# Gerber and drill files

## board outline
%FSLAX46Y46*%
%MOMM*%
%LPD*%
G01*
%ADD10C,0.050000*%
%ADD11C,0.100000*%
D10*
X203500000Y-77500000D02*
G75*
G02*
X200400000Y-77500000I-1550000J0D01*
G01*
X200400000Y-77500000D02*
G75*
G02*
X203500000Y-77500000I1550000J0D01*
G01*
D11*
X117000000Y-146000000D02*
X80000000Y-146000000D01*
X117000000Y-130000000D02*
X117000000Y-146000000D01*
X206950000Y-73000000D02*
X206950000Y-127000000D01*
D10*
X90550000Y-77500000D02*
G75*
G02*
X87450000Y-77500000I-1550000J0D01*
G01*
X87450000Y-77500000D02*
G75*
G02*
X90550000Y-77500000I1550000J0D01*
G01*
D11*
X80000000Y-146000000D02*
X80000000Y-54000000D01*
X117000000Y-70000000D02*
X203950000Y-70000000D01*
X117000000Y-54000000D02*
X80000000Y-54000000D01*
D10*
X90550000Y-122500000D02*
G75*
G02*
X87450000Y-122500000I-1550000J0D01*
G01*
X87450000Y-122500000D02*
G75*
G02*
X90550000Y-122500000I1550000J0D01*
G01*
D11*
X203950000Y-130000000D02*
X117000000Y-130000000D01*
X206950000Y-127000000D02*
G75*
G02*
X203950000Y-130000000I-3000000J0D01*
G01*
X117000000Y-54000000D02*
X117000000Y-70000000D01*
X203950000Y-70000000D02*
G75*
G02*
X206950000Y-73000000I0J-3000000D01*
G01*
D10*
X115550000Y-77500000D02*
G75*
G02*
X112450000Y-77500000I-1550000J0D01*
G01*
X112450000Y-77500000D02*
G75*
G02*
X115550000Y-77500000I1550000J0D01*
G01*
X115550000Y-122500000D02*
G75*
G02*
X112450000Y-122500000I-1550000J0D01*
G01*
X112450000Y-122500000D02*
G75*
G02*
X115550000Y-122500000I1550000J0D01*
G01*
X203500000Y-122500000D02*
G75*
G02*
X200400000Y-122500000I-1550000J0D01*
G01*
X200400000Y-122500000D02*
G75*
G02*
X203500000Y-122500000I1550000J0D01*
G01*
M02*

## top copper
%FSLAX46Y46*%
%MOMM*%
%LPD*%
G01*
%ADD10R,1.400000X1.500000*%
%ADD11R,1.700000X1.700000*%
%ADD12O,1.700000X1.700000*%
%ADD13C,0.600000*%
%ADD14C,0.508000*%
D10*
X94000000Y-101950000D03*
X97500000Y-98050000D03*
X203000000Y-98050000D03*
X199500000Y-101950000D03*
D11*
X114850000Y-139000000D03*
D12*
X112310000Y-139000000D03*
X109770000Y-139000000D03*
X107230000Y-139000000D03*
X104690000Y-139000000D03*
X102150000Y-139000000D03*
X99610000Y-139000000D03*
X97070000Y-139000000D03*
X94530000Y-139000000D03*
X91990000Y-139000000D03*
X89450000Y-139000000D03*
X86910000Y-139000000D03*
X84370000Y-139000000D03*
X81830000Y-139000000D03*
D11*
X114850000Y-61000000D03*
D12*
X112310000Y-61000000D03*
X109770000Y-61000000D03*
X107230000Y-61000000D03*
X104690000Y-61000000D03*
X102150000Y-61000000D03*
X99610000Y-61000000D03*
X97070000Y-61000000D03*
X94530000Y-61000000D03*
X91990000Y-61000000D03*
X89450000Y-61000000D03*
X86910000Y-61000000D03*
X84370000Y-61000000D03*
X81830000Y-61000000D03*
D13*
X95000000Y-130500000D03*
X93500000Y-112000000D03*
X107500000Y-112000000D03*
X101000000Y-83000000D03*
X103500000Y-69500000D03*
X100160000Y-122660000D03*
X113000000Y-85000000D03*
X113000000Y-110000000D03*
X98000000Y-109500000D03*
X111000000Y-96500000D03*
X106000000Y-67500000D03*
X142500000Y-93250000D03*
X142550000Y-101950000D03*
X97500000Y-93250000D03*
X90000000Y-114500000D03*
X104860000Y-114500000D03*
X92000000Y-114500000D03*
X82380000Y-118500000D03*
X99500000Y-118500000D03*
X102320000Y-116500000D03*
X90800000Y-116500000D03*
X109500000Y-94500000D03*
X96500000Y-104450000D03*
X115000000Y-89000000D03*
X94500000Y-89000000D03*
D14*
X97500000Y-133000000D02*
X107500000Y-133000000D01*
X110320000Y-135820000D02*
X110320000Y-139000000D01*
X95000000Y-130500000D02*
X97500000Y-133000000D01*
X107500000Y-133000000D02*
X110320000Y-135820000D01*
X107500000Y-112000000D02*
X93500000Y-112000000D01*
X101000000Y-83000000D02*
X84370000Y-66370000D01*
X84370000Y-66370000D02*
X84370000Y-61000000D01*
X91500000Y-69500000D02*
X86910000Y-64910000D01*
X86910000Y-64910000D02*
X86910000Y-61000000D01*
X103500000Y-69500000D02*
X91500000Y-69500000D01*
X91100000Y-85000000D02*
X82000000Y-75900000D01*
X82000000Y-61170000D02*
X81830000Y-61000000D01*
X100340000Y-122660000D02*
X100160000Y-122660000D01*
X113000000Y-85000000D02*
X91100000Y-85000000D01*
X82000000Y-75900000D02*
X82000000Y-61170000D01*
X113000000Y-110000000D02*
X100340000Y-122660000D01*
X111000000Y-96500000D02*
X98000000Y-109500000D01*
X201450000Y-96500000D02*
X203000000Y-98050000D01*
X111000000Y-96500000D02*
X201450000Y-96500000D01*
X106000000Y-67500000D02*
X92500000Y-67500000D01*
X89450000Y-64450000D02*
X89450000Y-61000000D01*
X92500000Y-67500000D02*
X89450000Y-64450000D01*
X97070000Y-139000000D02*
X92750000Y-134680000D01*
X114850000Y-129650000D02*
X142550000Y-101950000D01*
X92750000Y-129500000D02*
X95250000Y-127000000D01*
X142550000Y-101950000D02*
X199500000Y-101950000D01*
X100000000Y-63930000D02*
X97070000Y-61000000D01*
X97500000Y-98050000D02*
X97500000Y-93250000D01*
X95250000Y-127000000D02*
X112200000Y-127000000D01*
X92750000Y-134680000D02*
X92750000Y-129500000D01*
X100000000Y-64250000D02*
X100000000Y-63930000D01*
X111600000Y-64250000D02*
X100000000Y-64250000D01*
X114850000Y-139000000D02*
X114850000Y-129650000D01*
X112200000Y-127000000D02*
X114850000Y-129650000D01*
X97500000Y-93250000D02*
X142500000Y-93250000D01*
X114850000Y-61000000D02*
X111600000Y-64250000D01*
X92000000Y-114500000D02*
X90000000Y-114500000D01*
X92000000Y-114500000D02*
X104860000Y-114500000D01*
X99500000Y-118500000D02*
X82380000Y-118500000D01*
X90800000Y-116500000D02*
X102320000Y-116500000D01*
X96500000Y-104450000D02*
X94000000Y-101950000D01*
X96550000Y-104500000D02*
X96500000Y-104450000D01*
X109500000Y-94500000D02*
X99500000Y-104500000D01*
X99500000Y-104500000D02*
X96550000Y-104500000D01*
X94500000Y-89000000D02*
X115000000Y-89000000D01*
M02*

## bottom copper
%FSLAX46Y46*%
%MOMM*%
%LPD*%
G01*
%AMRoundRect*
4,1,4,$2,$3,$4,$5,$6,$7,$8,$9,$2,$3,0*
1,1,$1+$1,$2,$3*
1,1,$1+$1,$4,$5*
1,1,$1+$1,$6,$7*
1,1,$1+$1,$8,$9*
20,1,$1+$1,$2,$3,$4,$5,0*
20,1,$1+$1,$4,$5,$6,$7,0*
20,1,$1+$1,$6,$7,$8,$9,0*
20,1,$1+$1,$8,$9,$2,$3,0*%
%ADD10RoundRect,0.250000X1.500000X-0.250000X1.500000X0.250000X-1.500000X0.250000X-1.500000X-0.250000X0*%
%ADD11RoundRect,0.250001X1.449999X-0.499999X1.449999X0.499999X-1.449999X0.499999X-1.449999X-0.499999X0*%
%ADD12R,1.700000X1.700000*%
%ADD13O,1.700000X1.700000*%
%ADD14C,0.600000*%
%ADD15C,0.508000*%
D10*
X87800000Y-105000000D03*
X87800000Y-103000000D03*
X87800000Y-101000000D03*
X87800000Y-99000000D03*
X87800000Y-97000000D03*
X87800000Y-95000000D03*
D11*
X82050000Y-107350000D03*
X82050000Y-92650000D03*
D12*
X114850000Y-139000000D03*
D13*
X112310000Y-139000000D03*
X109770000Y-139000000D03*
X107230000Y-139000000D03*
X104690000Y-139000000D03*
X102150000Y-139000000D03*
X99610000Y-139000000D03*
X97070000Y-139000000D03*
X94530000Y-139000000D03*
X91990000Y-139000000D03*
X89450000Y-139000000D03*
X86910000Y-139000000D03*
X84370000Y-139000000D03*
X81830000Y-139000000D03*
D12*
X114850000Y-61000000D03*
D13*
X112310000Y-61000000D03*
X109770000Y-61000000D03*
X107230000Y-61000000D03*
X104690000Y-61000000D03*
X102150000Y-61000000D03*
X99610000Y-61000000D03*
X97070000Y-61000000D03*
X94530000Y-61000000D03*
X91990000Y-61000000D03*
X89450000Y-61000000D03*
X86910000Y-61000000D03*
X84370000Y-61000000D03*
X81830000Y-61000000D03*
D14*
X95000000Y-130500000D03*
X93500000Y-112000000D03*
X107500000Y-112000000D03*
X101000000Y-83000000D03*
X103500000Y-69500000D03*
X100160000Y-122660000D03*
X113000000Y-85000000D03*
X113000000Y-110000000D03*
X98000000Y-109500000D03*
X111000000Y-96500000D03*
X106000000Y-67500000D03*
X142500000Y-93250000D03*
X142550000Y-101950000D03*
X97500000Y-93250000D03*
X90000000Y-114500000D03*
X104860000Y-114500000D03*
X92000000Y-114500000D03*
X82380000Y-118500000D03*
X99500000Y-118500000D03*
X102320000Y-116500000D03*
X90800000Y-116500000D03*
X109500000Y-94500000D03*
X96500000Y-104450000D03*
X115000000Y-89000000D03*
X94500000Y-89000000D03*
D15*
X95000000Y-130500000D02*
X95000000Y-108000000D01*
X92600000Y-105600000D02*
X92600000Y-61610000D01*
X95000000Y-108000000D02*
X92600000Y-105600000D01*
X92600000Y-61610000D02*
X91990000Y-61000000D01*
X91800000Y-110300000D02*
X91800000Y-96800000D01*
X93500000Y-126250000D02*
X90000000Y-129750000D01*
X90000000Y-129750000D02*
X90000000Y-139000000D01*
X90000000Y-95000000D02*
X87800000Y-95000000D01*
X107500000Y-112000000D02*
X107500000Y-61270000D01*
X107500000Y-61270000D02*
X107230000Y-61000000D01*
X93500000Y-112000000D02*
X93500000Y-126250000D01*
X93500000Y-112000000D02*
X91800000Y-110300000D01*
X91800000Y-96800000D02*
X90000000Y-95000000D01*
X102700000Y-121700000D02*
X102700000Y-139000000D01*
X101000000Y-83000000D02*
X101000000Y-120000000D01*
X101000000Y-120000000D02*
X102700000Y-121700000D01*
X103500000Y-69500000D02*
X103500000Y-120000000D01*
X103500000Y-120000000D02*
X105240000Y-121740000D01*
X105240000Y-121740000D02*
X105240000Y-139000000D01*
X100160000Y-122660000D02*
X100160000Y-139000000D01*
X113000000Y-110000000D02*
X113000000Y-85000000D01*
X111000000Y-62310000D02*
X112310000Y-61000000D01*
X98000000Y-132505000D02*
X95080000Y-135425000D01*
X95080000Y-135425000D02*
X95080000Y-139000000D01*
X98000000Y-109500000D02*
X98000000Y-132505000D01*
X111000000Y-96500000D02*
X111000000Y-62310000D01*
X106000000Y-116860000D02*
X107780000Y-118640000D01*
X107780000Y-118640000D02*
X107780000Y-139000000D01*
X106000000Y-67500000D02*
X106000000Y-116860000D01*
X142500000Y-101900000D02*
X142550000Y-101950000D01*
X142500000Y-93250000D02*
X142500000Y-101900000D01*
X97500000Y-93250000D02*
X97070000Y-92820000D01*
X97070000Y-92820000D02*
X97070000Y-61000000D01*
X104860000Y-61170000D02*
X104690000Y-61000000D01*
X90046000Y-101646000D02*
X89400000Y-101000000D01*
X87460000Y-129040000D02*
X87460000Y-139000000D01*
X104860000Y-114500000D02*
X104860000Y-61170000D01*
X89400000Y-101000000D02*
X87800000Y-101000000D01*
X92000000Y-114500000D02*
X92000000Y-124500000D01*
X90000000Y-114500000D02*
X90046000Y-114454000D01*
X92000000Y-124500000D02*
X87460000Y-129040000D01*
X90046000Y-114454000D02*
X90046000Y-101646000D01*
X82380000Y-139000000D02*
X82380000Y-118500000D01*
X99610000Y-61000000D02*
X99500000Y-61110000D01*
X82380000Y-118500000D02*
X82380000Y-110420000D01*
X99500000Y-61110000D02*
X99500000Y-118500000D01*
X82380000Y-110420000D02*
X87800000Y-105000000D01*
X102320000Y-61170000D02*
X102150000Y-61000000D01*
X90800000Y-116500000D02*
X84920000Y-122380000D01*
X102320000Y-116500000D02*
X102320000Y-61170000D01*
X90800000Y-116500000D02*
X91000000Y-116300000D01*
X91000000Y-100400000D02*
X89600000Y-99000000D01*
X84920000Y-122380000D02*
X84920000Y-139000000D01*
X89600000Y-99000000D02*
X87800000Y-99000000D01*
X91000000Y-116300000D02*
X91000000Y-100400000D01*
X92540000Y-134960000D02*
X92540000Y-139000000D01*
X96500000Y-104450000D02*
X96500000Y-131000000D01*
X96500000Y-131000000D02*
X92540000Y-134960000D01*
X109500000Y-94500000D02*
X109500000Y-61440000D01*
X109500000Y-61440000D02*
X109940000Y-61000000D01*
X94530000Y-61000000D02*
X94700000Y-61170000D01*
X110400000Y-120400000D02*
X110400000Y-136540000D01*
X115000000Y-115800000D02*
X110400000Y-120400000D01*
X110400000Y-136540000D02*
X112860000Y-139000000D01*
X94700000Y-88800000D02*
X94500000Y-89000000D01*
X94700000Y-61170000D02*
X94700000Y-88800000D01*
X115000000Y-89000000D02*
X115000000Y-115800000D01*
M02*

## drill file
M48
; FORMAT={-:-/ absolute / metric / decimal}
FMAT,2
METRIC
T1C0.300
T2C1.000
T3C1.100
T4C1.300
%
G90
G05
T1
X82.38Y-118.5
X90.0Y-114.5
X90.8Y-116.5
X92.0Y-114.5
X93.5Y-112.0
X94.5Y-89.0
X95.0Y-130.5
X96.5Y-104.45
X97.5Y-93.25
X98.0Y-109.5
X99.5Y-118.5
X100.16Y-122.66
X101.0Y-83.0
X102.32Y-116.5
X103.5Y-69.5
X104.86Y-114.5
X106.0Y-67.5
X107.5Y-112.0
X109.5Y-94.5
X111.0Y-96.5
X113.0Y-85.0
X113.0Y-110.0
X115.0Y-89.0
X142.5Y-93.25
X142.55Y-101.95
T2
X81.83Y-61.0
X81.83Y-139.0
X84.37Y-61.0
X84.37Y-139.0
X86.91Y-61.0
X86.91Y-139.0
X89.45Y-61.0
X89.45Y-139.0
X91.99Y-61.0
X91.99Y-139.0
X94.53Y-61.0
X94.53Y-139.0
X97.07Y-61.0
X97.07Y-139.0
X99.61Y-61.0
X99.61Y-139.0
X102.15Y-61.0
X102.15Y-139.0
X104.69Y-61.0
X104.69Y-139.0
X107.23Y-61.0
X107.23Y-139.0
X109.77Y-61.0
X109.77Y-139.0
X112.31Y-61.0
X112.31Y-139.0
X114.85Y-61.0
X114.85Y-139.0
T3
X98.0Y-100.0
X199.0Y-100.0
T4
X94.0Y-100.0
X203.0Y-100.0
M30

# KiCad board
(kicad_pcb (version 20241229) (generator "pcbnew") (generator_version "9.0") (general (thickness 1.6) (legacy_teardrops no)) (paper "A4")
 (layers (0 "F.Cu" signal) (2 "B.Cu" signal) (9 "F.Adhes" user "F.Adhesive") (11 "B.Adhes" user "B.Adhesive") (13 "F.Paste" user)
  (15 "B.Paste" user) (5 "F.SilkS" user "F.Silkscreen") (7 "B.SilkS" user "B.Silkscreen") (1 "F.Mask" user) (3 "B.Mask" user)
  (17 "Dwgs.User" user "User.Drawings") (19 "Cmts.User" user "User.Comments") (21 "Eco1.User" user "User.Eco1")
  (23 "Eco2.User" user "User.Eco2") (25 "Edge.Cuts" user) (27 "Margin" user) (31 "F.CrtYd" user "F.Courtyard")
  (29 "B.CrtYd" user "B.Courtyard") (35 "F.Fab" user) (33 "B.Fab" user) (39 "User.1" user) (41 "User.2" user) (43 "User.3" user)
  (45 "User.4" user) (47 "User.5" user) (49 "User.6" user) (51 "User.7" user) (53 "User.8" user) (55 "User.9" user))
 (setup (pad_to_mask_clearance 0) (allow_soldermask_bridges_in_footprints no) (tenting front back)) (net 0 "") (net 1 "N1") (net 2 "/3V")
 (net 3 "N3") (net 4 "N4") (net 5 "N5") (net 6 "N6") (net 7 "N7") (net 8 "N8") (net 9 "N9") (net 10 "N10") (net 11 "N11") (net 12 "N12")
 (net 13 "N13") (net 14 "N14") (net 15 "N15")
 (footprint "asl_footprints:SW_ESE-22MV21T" (layer "F.Cu") (at 96 100 180)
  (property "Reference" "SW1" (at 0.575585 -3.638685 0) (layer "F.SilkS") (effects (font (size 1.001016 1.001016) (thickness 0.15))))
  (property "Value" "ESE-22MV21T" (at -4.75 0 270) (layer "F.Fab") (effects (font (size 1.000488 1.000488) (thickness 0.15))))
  (pad "" np_thru_hole circle (at -2 0 180) (size 1.1 1.1) (drill 1.1) (layers "*.Cu" "*.Mask"))
  (pad "" np_thru_hole circle (at 2 0 180) (size 1.3 1.3) (drill 1.3) (layers "*.Cu" "*.Mask"))
  (pad "1" smd rect (at 2 -1.95 180) (size 1.4 1.5) (layers "F.Cu" "F.Mask" "F.Paste") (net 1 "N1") (solder_mask_margin 0.102))
  (pad "2" smd rect (at -1.5 1.95 180) (size 1.4 1.5) (layers "F.Cu" "F.Mask" "F.Paste") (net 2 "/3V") (solder_mask_margin 0.102)))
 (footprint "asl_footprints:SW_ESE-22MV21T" (layer "F.Cu") (at 201 100)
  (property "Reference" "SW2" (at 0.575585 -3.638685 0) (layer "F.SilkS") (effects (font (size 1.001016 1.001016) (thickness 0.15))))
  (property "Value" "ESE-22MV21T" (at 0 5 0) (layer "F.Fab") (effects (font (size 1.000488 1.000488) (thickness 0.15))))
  (pad "" np_thru_hole circle (at -2 0) (size 1.1 1.1) (drill 1.1) (layers "*.Cu" "*.Mask"))
  (pad "" np_thru_hole circle (at 2 0) (size 1.3 1.3) (drill 1.3) (layers "*.Cu" "*.Mask"))
  (pad "1" smd rect (at 2 -1.95) (size 1.4 1.5) (layers "F.Cu" "F.Mask" "F.Paste") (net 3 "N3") (solder_mask_margin 0.102))
  (pad "2" smd rect (at -1.5 1.95) (size 1.4 1.5) (layers "F.Cu" "F.Mask" "F.Paste") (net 2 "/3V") (solder_mask_margin 0.102)))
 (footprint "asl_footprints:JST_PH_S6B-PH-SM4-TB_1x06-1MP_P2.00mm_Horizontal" (layer "B.Cu") (at 84.95 100 90)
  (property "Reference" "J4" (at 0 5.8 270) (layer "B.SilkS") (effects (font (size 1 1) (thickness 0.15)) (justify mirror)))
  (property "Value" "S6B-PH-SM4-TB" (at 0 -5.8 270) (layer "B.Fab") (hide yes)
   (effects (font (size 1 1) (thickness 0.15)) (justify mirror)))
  (pad "1" smd roundrect (at -5 2.85 90) (size 1 3.5) (layers "B.Cu" "B.Mask" "B.Paste") (roundrect_rratio 0.25) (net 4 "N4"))
  (pad "2" smd roundrect (at -3 2.85 90) (size 1 3.5) (layers "B.Cu" "B.Mask" "B.Paste") (roundrect_rratio 0.25) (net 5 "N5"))
  (pad "3" smd roundrect (at -1 2.85 90) (size 1 3.5) (layers "B.Cu" "B.Mask" "B.Paste") (roundrect_rratio 0.25) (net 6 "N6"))
  (pad "4" smd roundrect (at 1 2.85 90) (size 1 3.5) (layers "B.Cu" "B.Mask" "B.Paste") (roundrect_rratio 0.25) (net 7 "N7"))
  (pad "5" smd roundrect (at 3 2.85 90) (size 1 3.5) (layers "B.Cu" "B.Mask" "B.Paste") (roundrect_rratio 0.25) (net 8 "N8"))
  (pad "6" smd roundrect (at 5 2.85 90) (size 1 3.5) (layers "B.Cu" "B.Mask" "B.Paste") (roundrect_rratio 0.25) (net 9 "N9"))
  (pad "MP" smd roundrect (at -7.35 -2.9 90) (size 1.5 3.4) (layers "B.Cu" "B.Mask" "B.Paste") (roundrect_rratio 0.166667))
  (pad "MP" smd roundrect (at 7.35 -2.9 90) (size 1.5 3.4) (layers "B.Cu" "B.Mask" "B.Paste") (roundrect_rratio 0.166667)))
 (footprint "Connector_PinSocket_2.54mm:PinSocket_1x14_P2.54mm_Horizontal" (layer "B.Cu") (at 114.85 139 90)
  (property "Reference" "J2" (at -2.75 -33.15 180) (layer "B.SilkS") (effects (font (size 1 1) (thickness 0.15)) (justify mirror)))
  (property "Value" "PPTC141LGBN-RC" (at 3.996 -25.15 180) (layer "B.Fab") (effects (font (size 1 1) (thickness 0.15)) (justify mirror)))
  (pad "1" thru_hole rect (at 0 0 90) (size 1.7 1.7) (drill 1) (layers "*.Cu" "*.Mask") (remove_unused_layers no) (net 2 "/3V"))
  (pad "2" thru_hole oval (at 0 -2.54 90) (size 1.7 1.7) (drill 1) (layers "*.Cu" "*.Mask") (remove_unused_layers no) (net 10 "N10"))
  (pad "3" thru_hole oval (at 0 -5.08 90) (size 1.7 1.7) (drill 1) (layers "*.Cu" "*.Mask") (remove_unused_layers no) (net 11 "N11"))
  (pad "4" thru_hole oval (at 0 -7.62 90) (size 1.7 1.7) (drill 1) (layers "*.Cu" "*.Mask") (remove_unused_layers no) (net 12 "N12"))
  (pad "5" thru_hole oval (at 0 -10.16 90) (size 1.7 1.7) (drill 1) (layers "*.Cu" "*.Mask") (remove_unused_layers no) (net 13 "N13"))
  (pad "6" thru_hole oval (at 0 -12.7 90) (size 1.7 1.7) (drill 1) (layers "*.Cu" "*.Mask") (remove_unused_layers no) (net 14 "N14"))
  (pad "7" thru_hole oval (at 0 -15.24 90) (size 1.7 1.7) (drill 1) (layers "*.Cu" "*.Mask") (remove_unused_layers no) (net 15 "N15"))
  (pad "8" thru_hole oval (at 0 -17.78 90) (size 1.7 1.7) (drill 1) (layers "*.Cu" "*.Mask") (remove_unused_layers no) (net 2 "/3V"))
  (pad "9" thru_hole oval (at 0 -20.32 90) (size 1.7 1.7) (drill 1) (layers "*.Cu" "*.Mask") (remove_unused_layers no) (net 3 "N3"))
  (pad "10" thru_hole oval (at 0 -22.86 90) (size 1.7 1.7) (drill 1) (layers "*.Cu" "*.Mask") (remove_unused_layers no) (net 1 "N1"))
  (pad "11" thru_hole oval (at 0 -25.4 90) (size 1.7 1.7) (drill 1) (layers "*.Cu" "*.Mask") (remove_unused_layers no) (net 9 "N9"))
  (pad "12" thru_hole oval (at 0 -27.94 90) (size 1.7 1.7) (drill 1) (layers "*.Cu" "*.Mask") (remove_unused_layers no) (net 6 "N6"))
  (pad "13" thru_hole oval (at 0 -30.48 90) (size 1.7 1.7) (drill 1) (layers "*.Cu" "*.Mask") (remove_unused_layers no) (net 7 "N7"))
  (pad "14" thru_hole oval (at 0 -33.02 90) (size 1.7 1.7) (drill 1) (layers "*.Cu" "*.Mask") (remove_unused_layers no) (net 4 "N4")))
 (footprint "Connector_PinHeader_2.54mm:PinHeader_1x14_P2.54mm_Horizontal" (layer "B.Cu") (at 114.85 61 90)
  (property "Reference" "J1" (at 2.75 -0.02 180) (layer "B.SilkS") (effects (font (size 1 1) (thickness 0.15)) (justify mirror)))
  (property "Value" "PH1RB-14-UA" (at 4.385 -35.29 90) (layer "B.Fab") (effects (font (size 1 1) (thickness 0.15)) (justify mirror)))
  (pad "1" thru_hole rect (at 0 0 90) (size 1.7 1.7) (drill 1) (layers "*.Cu" "*.Mask") (remove_unused_layers no) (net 2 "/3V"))
  (pad "2" thru_hole oval (at 0 -2.54 90) (size 1.7 1.7) (drill 1) (layers "*.Cu" "*.Mask") (remove_unused_layers no) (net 3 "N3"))
  (pad "3" thru_hole oval (at 0 -5.08 90) (size 1.7 1.7) (drill 1) (layers "*.Cu" "*.Mask") (remove_unused_layers no) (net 1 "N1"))
  (pad "4" thru_hole oval (at 0 -7.62 90) (size 1.7 1.7) (drill 1) (layers "*.Cu" "*.Mask") (remove_unused_layers no) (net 9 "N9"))
  (pad "5" thru_hole oval (at 0 -10.16 90) (size 1.7 1.7) (drill 1) (layers "*.Cu" "*.Mask") (remove_unused_layers no) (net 6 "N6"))
  (pad "6" thru_hole oval (at 0 -12.7 90) (size 1.7 1.7) (drill 1) (layers "*.Cu" "*.Mask") (remove_unused_layers no) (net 7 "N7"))
  (pad "7" thru_hole oval (at 0 -15.24 90) (size 1.7 1.7) (drill 1) (layers "*.Cu" "*.Mask") (remove_unused_layers no) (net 4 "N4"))
  (pad "8" thru_hole oval (at 0 -17.78 90) (size 1.7 1.7) (drill 1) (layers "*.Cu" "*.Mask") (remove_unused_layers no) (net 2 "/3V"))
  (pad "9" thru_hole oval (at 0 -20.32 90) (size 1.7 1.7) (drill 1) (layers "*.Cu" "*.Mask") (remove_unused_layers no) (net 10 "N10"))
  (pad "10" thru_hole oval (at 0 -22.86 90) (size 1.7 1.7) (drill 1) (layers "*.Cu" "*.Mask") (remove_unused_layers no) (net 11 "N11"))
  (pad "11" thru_hole oval (at 0 -25.4 90) (size 1.7 1.7) (drill 1) (layers "*.Cu" "*.Mask") (remove_unused_layers no) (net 12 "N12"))
  (pad "12" thru_hole oval (at 0 -27.94 90) (size 1.7 1.7) (drill 1) (layers "*.Cu" "*.Mask") (remove_unused_layers no) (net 13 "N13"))
  (pad "13" thru_hole oval (at 0 -30.48 90) (size 1.7 1.7) (drill 1) (layers "*.Cu" "*.Mask") (remove_unused_layers no) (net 14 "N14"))
  (pad "14" thru_hole oval (at 0 -33.02 90) (size 1.7 1.7) (drill 1) (layers "*.Cu" "*.Mask") (remove_unused_layers no) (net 15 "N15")))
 (gr_circle (center 201.95 77.5) (end 203.5 77.5) (stroke (width 0.05) (type default)) (fill no) (layer "Edge.Cuts"))
 (gr_line (start 117 146) (end 80 146) (stroke (width 0.1) (type default)) (layer "Edge.Cuts"))
 (gr_line (start 117 130) (end 117 146) (stroke (width 0.1) (type default)) (layer "Edge.Cuts"))
 (gr_line (start 206.95 73) (end 206.95 127) (stroke (width 0.1) (type default)) (layer "Edge.Cuts"))
 (gr_circle (center 89 77.5) (end 90.55 77.5) (stroke (width 0.05) (type default)) (fill no) (layer "Edge.Cuts"))
 (gr_line (start 80 146) (end 80 54) (stroke (width 0.1) (type default)) (layer "Edge.Cuts"))
 (gr_line (start 117 70) (end 203.95 70) (stroke (width 0.1) (type default)) (layer "Edge.Cuts"))
 (gr_line (start 117 54) (end 80 54) (stroke (width 0.1) (type default)) (layer "Edge.Cuts"))
 (gr_circle (center 89 122.5) (end 90.55 122.5) (stroke (width 0.05) (type default)) (fill no) (layer "Edge.Cuts"))
 (gr_line (start 203.95 130) (end 117 130) (stroke (width 0.1) (type default)) (layer "Edge.Cuts"))
 (gr_arc (start 206.95 127) (mid 206.07132 129.12132) (end 203.95 130) (stroke (width 0.1) (type default)) (layer "Edge.Cuts"))
 (gr_line (start 117 54) (end 117 70) (stroke (width 0.1) (type default)) (layer "Edge.Cuts"))
 (gr_arc (start 203.95 70) (mid 206.07132 70.87868) (end 206.95 73) (stroke (width 0.1) (type default)) (layer "Edge.Cuts"))
 (gr_circle (center 114 77.5) (end 115.55 77.5) (stroke (width 0.05) (type default)) (fill no) (layer "Edge.Cuts"))
 (gr_circle (center 114 122.5) (end 115.55 122.5) (stroke (width 0.05) (type default)) (fill no) (layer "Edge.Cuts"))
 (gr_circle (center 201.95 122.5) (end 203.5 122.5) (stroke (width 0.05) (type default)) (fill no) (layer "Edge.Cuts"))
 (segment (start 97.5 133) (end 107.5 133) (width 0.508) (layer "F.Cu") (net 11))
 (segment (start 110.32 135.82) (end 110.32 139) (width 0.508) (layer "F.Cu") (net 11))
 (segment (start 95 130.5) (end 97.5 133) (width 0.508) (layer "F.Cu") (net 11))
 (segment (start 107.5 133) (end 110.32 135.82) (width 0.508) (layer "F.Cu") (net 11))
 (via (at 95 130.5) (size 0.6) (drill 0.3) (layers "F.Cu" "B.Cu") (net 11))
 (segment (start 95 130.5) (end 95 108) (width 0.508) (layer "B.Cu") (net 11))
 (segment (start 92.6 105.6) (end 92.6 61.61) (width 0.508) (layer "B.Cu") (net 11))
 (segment (start 95 108) (end 92.6 105.6) (width 0.508) (layer "B.Cu") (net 11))
 (segment (start 92.6 61.61) (end 91.99 61) (width 0.508) (layer "B.Cu") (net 11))
 (segment (start 107.5 112) (end 93.5 112) (width 0.508) (layer "F.Cu") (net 9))
 (via (at 93.5 112) (size 0.6) (drill 0.3) (layers "F.Cu" "B.Cu") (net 9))
 (via (at 107.5 112) (size 0.6) (drill 0.3) (layers "F.Cu" "B.Cu") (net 9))
 (segment (start 91.8 110.3) (end 91.8 96.8) (width 0.508) (layer "B.Cu") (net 9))
 (segment (start 93.5 126.25) (end 90 129.75) (width 0.508) (layer "B.Cu") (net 9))
 (segment (start 90 129.75) (end 90 139) (width 0.508) (layer "B.Cu") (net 9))
 (segment (start 90 95) (end 87.8 95) (width 0.508) (layer "B.Cu") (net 9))
 (segment (start 107.5 112) (end 107.5 61.27) (width 0.508) (layer "B.Cu") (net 9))
 (segment (start 107.5 61.27) (end 107.23 61) (width 0.508) (layer "B.Cu") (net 9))
 (segment (start 93.5 112) (end 93.5 126.25) (width 0.508) (layer "B.Cu") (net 9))
 (segment (start 93.5 112) (end 91.8 110.3) (width 0.508) (layer "B.Cu") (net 9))
 (segment (start 91.8 96.8) (end 90 95) (width 0.508) (layer "B.Cu") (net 9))
 (segment (start 101 83) (end 84.37 66.37) (width 0.508) (layer "F.Cu") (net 14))
 (segment (start 84.37 66.37) (end 84.37 61) (width 0.508) (layer "F.Cu") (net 14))
 (via (at 101 83) (size 0.6) (drill 0.3) (layers "F.Cu" "B.Cu") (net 14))
 (segment (start 102.7 121.7) (end 102.7 139) (width 0.508) (layer "B.Cu") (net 14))
 (segment (start 101 83) (end 101 120) (width 0.508) (layer "B.Cu") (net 14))
 (segment (start 101 120) (end 102.7 121.7) (width 0.508) (layer "B.Cu") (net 14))
 (segment (start 91.5 69.5) (end 86.91 64.91) (width 0.508) (layer "F.Cu") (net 13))
 (segment (start 86.91 64.91) (end 86.91 61) (width 0.508) (layer "F.Cu") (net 13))
 (segment (start 103.5 69.5) (end 91.5 69.5) (width 0.508) (layer "F.Cu") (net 13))
 (via (at 103.5 69.5) (size 0.6) (drill 0.3) (layers "F.Cu" "B.Cu") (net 13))
 (segment (start 103.5 69.5) (end 103.5 120) (width 0.508) (layer "B.Cu") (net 13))
 (segment (start 103.5 120) (end 105.24 121.74) (width 0.508) (layer "B.Cu") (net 13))
 (segment (start 105.24 121.74) (end 105.24 139) (width 0.508) (layer "B.Cu") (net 13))
 (segment (start 91.1 85) (end 82 75.9) (width 0.508) (layer "F.Cu") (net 15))
 (segment (start 82 61.17) (end 81.83 61) (width 0.508) (layer "F.Cu") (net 15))
 (segment (start 100.34 122.66) (end 100.16 122.66) (width 0.508) (layer "F.Cu") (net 15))
 (segment (start 113 85) (end 91.1 85) (width 0.508) (layer "F.Cu") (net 15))
 (segment (start 82 75.9) (end 82 61.17) (width 0.508) (layer "F.Cu") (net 15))
 (segment (start 113 110) (end 100.34 122.66) (width 0.508) (layer "F.Cu") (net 15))
 (via (at 100.16 122.66) (size 0.6) (drill 0.3) (layers "F.Cu" "B.Cu") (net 15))
 (via (at 113 85) (size 0.6) (drill 0.3) (layers "F.Cu" "B.Cu") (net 15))
 (via (at 113 110) (size 0.6) (drill 0.3) (layers "F.Cu" "B.Cu") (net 15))
 (segment (start 100.16 122.66) (end 100.16 139) (width 0.508) (layer "B.Cu") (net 15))
 (segment (start 113 110) (end 113 85) (width 0.508) (layer "B.Cu") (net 15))
 (segment (start 111 96.5) (end 98 109.5) (width 0.508) (layer "F.Cu") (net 3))
 (segment (start 201.45 96.5) (end 203 98.05) (width 0.508) (layer "F.Cu") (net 3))
 (segment (start 111 96.5) (end 201.45 96.5) (width 0.508) (layer "F.Cu") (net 3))
 (via (at 98 109.5) (size 0.6) (drill 0.3) (layers "F.Cu" "B.Cu") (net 3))
 (via (at 111 96.5) (size 0.6) (drill 0.3) (layers "F.Cu" "B.Cu") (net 3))
 (segment (start 111 62.31) (end 112.31 61) (width 0.508) (layer "B.Cu") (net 3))
 (segment (start 98 132.505) (end 95.08 135.425) (width 0.508) (layer "B.Cu") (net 3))
 (segment (start 95.08 135.425) (end 95.08 139) (width 0.508) (layer "B.Cu") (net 3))
 (segment (start 98 109.5) (end 98 132.505) (width 0.508) (layer "B.Cu") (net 3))
 (segment (start 111 96.5) (end 111 62.31) (width 0.508) (layer "B.Cu") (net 3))
 (segment (start 106 67.5) (end 92.5 67.5) (width 0.508) (layer "F.Cu") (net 12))
 (segment (start 89.45 64.45) (end 89.45 61) (width 0.508) (layer "F.Cu") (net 12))
 (segment (start 92.5 67.5) (end 89.45 64.45) (width 0.508) (layer "F.Cu") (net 12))
 (via (at 106 67.5) (size 0.6) (drill 0.3) (layers "F.Cu" "B.Cu") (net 12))
 (segment (start 106 116.86) (end 107.78 118.64) (width 0.508) (layer "B.Cu") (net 12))
 (segment (start 107.78 118.64) (end 107.78 139) (width 0.508) (layer "B.Cu") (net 12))
 (segment (start 106 67.5) (end 106 116.86) (width 0.508) (layer "B.Cu") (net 12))
 (segment (start 97.07 139) (end 92.75 134.68) (width 0.508) (layer "F.Cu") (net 2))
 (segment (start 114.85 129.65) (end 142.55 101.95) (width 0.508) (layer "F.Cu") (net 2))
 (segment (start 92.75 129.5) (end 95.25 127) (width 0.508) (layer "F.Cu") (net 2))
 (segment (start 142.55 101.95) (end 199.5 101.95) (width 0.508) (layer "F.Cu") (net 2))
 (segment (start 100 63.93) (end 97.07 61) (width 0.508) (layer "F.Cu") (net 2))
 (segment (start 97.5 98.05) (end 97.5 93.25) (width 0.508) (layer "F.Cu") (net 2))
 (segment (start 95.25 127) (end 112.2 127) (width 0.508) (layer "F.Cu") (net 2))
 (segment (start 92.75 134.68) (end 92.75 129.5) (width 0.508) (layer "F.Cu") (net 2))
 (segment (start 100 64.25) (end 100 63.93) (width 0.508) (layer "F.Cu") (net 2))
 (segment (start 111.6 64.25) (end 100 64.25) (width 0.508) (layer "F.Cu") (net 2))
 (segment (start 114.85 139) (end 114.85 129.65) (width 0.508) (layer "F.Cu") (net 2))
 (segment (start 112.2 127) (end 114.85 129.65) (width 0.508) (layer "F.Cu") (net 2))
 (segment (start 97.5 93.25) (end 142.5 93.25) (width 0.508) (layer "F.Cu") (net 2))
 (segment (start 114.85 61) (end 111.6 64.25) (width 0.508) (layer "F.Cu") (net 2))
 (via (at 142.5 93.25) (size 0.6) (drill 0.3) (layers "F.Cu" "B.Cu") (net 2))
 (via (at 142.55 101.95) (size 0.6) (drill 0.3) (layers "F.Cu" "B.Cu") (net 2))
 (via (at 97.5 93.25) (size 0.6) (drill 0.3) (layers "F.Cu" "B.Cu") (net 2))
 (segment (start 142.5 101.9) (end 142.55 101.95) (width 0.508) (layer "B.Cu") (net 2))
 (segment (start 142.5 93.25) (end 142.5 101.9) (width 0.508) (layer "B.Cu") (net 2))
 (segment (start 97.5 93.25) (end 97.07 92.82) (width 0.508) (layer "B.Cu") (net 2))
 (segment (start 97.07 92.82) (end 97.07 61) (width 0.508) (layer "B.Cu") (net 2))
 (segment (start 92 114.5) (end 90 114.5) (width 0.508) (layer "F.Cu") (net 6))
 (segment (start 92 114.5) (end 104.86 114.5) (width 0.508) (layer "F.Cu") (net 6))
 (via (at 90 114.5) (size 0.6) (drill 0.3) (layers "F.Cu" "B.Cu") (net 6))
 (via (at 104.86 114.5) (size 0.6) (drill 0.3) (layers "F.Cu" "B.Cu") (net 6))
 (via (at 92 114.5) (size 0.6) (drill 0.3) (layers "F.Cu" "B.Cu") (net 6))
 (segment (start 104.86 61.17) (end 104.69 61) (width 0.508) (layer "B.Cu") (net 6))
 (segment (start 90.046 101.646) (end 89.4 101) (width 0.508) (layer "B.Cu") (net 6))
 (segment (start 87.46 129.04) (end 87.46 139) (width 0.508) (layer "B.Cu") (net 6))
 (segment (start 104.86 114.5) (end 104.86 61.17) (width 0.508) (layer "B.Cu") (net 6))
 (segment (start 89.4 101) (end 87.8 101) (width 0.508) (layer "B.Cu") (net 6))
 (segment (start 92 114.5) (end 92 124.5) (width 0.508) (layer "B.Cu") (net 6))
 (segment (start 90 114.5) (end 90.046 114.454) (width 0.508) (layer "B.Cu") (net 6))
 (segment (start 92 124.5) (end 87.46 129.04) (width 0.508) (layer "B.Cu") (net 6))
 (segment (start 90.046 114.454) (end 90.046 101.646) (width 0.508) (layer "B.Cu") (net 6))
 (segment (start 99.5 118.5) (end 82.38 118.5) (width 0.508) (layer "F.Cu") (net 4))
 (via (at 82.38 118.5) (size 0.6) (drill 0.3) (layers "F.Cu" "B.Cu") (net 4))
 (via (at 99.5 118.5) (size 0.6) (drill 0.3) (layers "F.Cu" "B.Cu") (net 4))
 (segment (start 82.38 139) (end 82.38 118.5) (width 0.508) (layer "B.Cu") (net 4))
 (segment (start 99.61 61) (end 99.5 61.11) (width 0.508) (layer "B.Cu") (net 4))
 (segment (start 82.38 118.5) (end 82.38 110.42) (width 0.508) (layer "B.Cu") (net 4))
 (segment (start 99.5 61.11) (end 99.5 118.5) (width 0.508) (layer "B.Cu") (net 4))
 (segment (start 82.38 110.42) (end 87.8 105) (width 0.508) (layer "B.Cu") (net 4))
 (segment (start 90.8 116.5) (end 102.32 116.5) (width 0.508) (layer "F.Cu") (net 7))
 (via (at 102.32 116.5) (size 0.6) (drill 0.3) (layers "F.Cu" "B.Cu") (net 7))
 (via (at 90.8 116.5) (size 0.6) (drill 0.3) (layers "F.Cu" "B.Cu") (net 7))
 (segment (start 102.32 61.17) (end 102.15 61) (width 0.508) (layer "B.Cu") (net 7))
 (segment (start 90.8 116.5) (end 84.92 122.38) (width 0.508) (layer "B.Cu") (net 7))
 (segment (start 102.32 116.5) (end 102.32 61.17) (width 0.508) (layer "B.Cu") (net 7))
 (segment (start 90.8 116.5) (end 91 116.3) (width 0.508) (layer "B.Cu") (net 7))
 (segment (start 91 100.4) (end 89.6 99) (width 0.508) (layer "B.Cu") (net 7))
 (segment (start 84.92 122.38) (end 84.92 139) (width 0.508) (layer "B.Cu") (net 7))
 (segment (start 89.6 99) (end 87.8 99) (width 0.508) (layer "B.Cu") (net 7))
 (segment (start 91 116.3) (end 91 100.4) (width 0.508) (layer "B.Cu") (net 7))
 (segment (start 96.5 104.45) (end 94 101.95) (width 0.508) (layer "F.Cu") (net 1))
 (segment (start 96.55 104.5) (end 96.5 104.45) (width 0.508) (layer "F.Cu") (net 1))
 (segment (start 109.5 94.5) (end 99.5 104.5) (width 0.508) (layer "F.Cu") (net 1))
 (segment (start 99.5 104.5) (end 96.55 104.5) (width 0.508) (layer "F.Cu") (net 1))
 (via (at 109.5 94.5) (size 0.6) (drill 0.3) (layers "F.Cu" "B.Cu") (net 1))
 (via (at 96.5 104.45) (size 0.6) (drill 0.3) (layers "F.Cu" "B.Cu") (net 1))
 (segment (start 92.54 134.96) (end 92.54 139) (width 0.508) (layer "B.Cu") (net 1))
 (segment (start 96.5 104.45) (end 96.5 131) (width 0.508) (layer "B.Cu") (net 1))
 (segment (start 96.5 131) (end 92.54 134.96) (width 0.508) (layer "B.Cu") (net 1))
 (segment (start 109.5 94.5) (end 109.5 61.44) (width 0.508) (layer "B.Cu") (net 1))
 (segment (start 109.5 61.44) (end 109.94 61) (width 0.508) (layer "B.Cu") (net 1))
 (segment (start 94.5 89) (end 115 89) (width 0.508) (layer "F.Cu") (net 10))
 (via (at 115 89) (size 0.6) (drill 0.3) (layers "F.Cu" "B.Cu") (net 10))
 (via (at 94.5 89) (size 0.6) (drill 0.3) (layers "F.Cu" "B.Cu") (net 10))
 (segment (start 94.53 61) (end 94.7 61.17) (width 0.508) (layer "B.Cu") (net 10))
 (segment (start 110.4 120.4) (end 110.4 136.54) (width 0.508) (layer "B.Cu") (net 10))
 (segment (start 115 115.8) (end 110.4 120.4) (width 0.508) (layer "B.Cu") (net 10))
 (segment (start 110.4 136.54) (end 112.86 139) (width 0.508) (layer "B.Cu") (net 10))
 (segment (start 94.7 88.8) (end 94.5 89) (width 0.508) (layer "B.Cu") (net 10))
 (segment (start 94.7 61.17) (end 94.7 88.8) (width 0.508) (layer "B.Cu") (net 10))
 (segment (start 115 89) (end 115 115.8) (width 0.508) (layer "B.Cu") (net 10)))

